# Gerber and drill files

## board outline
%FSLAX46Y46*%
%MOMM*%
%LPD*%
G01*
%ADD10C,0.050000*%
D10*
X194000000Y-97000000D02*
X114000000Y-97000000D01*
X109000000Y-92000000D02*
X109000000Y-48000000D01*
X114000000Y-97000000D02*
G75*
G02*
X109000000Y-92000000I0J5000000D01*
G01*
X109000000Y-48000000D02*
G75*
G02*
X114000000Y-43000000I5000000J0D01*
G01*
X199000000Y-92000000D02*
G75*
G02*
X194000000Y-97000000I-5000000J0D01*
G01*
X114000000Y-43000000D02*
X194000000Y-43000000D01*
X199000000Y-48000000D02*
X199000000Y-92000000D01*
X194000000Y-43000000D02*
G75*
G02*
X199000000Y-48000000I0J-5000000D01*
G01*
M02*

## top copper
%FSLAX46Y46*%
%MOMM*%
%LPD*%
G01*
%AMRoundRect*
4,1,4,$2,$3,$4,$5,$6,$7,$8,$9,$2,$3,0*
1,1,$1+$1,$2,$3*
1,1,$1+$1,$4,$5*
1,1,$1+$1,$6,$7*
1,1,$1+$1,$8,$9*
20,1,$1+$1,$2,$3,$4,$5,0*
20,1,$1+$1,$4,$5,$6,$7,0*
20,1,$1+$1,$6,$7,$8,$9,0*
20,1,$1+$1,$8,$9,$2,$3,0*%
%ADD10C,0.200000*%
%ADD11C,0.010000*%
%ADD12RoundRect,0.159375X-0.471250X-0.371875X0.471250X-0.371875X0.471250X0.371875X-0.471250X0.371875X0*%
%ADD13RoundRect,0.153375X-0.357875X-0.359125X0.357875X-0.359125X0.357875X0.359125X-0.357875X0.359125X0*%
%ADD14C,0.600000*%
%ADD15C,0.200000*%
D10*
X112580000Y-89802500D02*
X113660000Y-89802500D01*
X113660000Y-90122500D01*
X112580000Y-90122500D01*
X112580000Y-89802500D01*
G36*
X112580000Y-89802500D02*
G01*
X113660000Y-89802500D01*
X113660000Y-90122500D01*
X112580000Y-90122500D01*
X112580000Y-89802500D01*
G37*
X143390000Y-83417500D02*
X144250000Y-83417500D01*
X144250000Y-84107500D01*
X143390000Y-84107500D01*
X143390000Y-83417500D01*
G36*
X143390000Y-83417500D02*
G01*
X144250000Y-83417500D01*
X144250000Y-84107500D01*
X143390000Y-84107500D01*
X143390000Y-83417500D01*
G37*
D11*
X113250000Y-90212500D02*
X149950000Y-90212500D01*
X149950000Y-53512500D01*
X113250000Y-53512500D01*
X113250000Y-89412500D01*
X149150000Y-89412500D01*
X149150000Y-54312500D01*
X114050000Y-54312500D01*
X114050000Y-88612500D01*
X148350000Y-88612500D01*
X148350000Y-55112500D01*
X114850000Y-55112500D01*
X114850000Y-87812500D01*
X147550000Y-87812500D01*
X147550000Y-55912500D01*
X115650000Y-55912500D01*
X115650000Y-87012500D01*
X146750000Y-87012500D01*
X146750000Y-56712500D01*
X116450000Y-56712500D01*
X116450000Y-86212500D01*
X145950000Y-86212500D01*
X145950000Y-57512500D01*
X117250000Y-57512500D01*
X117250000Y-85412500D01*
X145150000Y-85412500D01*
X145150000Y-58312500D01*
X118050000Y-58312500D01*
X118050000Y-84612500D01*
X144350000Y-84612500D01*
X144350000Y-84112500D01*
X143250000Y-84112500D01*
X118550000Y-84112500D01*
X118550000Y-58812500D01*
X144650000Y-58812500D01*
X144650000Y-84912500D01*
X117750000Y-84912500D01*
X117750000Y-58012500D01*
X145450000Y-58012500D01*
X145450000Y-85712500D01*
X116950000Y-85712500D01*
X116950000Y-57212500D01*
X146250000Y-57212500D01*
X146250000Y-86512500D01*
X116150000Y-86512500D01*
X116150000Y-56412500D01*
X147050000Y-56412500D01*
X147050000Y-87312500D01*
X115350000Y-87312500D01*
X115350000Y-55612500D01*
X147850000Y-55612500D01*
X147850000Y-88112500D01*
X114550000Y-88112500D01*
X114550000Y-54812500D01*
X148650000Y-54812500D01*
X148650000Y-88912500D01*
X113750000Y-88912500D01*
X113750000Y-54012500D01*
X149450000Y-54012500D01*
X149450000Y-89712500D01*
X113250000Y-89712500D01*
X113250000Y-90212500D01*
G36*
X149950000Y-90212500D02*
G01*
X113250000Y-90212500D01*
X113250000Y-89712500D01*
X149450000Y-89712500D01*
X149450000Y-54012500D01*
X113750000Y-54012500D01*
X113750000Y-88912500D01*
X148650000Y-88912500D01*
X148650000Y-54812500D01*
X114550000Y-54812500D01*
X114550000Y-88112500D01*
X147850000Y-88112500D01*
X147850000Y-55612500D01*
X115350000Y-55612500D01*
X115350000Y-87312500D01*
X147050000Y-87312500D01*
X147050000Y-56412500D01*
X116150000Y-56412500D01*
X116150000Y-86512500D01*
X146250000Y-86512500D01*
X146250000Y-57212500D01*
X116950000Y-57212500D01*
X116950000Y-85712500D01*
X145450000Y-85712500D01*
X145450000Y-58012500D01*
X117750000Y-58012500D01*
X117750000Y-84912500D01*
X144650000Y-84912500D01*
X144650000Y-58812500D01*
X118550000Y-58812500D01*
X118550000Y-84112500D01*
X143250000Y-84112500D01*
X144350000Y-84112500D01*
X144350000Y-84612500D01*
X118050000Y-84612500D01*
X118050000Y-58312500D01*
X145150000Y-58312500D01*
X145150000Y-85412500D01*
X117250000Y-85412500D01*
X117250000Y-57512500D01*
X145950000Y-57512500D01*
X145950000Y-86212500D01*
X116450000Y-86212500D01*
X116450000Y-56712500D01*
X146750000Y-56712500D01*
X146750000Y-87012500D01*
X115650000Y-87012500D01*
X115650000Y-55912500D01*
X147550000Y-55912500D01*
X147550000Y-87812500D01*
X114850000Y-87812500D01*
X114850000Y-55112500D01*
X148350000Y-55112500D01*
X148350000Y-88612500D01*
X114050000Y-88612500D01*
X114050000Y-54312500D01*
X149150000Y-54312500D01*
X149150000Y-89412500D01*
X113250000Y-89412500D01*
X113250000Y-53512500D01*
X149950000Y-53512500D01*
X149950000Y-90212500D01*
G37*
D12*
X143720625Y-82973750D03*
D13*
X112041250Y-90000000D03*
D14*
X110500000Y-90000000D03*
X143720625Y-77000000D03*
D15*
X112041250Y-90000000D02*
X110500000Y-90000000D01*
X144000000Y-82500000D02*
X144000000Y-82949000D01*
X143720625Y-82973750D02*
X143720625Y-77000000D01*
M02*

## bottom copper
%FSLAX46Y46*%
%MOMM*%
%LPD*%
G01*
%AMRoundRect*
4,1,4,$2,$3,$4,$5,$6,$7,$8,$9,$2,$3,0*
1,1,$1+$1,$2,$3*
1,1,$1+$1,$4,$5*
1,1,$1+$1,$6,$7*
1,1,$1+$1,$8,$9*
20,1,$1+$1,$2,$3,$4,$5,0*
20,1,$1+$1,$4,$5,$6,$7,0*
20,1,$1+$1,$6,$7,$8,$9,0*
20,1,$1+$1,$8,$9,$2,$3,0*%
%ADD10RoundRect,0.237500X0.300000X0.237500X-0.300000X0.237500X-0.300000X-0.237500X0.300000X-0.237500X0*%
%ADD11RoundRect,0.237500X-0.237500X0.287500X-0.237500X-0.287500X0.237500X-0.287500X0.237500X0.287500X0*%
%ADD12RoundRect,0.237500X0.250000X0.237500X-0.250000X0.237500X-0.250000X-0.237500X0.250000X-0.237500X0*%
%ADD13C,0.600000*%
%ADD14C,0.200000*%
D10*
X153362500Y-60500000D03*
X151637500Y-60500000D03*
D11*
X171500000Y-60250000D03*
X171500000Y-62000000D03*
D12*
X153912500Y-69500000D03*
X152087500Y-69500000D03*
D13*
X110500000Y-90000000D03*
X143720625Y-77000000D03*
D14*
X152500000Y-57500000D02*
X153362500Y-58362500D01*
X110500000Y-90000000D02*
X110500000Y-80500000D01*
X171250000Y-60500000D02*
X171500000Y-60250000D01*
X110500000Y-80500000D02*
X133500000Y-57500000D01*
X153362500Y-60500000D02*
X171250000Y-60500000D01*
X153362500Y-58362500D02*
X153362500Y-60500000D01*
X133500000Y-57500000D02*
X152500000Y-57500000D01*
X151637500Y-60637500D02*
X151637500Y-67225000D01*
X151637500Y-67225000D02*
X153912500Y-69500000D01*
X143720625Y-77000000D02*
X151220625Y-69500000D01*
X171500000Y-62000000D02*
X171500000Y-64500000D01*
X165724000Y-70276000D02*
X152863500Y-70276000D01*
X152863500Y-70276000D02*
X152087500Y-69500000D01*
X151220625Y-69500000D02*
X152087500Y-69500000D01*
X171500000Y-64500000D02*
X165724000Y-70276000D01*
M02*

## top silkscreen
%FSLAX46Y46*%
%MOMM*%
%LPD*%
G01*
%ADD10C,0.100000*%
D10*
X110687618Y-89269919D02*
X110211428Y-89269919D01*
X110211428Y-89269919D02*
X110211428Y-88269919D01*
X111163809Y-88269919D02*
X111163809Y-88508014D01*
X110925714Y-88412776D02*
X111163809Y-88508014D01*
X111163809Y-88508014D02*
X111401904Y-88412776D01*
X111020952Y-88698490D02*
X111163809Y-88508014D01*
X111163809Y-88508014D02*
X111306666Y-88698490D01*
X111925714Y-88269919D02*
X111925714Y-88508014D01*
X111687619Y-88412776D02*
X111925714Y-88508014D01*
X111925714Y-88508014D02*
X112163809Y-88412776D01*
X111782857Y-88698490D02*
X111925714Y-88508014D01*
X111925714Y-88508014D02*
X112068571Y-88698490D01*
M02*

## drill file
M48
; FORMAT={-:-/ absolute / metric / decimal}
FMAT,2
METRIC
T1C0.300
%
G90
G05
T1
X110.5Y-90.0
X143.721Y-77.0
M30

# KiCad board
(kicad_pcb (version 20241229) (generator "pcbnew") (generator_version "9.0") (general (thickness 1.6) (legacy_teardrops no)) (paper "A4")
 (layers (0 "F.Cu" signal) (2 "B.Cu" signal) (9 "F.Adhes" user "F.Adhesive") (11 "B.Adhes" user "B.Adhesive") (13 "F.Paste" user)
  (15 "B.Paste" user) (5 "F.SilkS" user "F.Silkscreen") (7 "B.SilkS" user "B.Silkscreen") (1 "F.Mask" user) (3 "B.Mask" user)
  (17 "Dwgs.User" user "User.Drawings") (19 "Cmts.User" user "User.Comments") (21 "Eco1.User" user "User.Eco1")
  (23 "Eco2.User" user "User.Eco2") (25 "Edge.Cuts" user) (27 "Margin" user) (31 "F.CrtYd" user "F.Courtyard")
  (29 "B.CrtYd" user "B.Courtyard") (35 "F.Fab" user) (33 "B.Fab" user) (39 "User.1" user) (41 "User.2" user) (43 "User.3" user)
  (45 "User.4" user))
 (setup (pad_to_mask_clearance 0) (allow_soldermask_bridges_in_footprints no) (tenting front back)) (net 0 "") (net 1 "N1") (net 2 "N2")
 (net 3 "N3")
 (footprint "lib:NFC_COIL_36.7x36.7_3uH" (layer "F.Cu") (at 113.25 90.2125)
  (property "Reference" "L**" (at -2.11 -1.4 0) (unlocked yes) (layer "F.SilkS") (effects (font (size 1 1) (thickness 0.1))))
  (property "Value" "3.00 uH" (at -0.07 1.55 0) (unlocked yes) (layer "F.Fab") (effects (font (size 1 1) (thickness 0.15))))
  (fp_rect (start -0.67 -0.41) (end 0.41 -0.09) (stroke (width 0.2) (type solid)) (fill yes) (layer "F.Cu"))
  (fp_rect (start 30.14 -6.795) (end 31 -6.105) (stroke (width 0.2) (type solid)) (fill yes) (layer "F.Cu"))
  (fp_poly
   (pts (xy 0 0) (xy 36.7 0) (xy 36.7 -36.7) (xy 0 -36.7) (xy 0 -0.8) (xy 35.9 -0.8) (xy 35.9 -35.9) (xy 0.8 -35.9) (xy 0.8 -1.6)
    (xy 35.1 -1.6) (xy 35.1 -35.1) (xy 1.6 -35.1) (xy 1.6 -2.4) (xy 34.3 -2.4) (xy 34.3 -34.3) (xy 2.4 -34.3) (xy 2.4 -3.2) (xy 33.5 -3.2)
    (xy 33.5 -33.5) (xy 3.2 -33.5) (xy 3.2 -4) (xy 32.7 -4) (xy 32.7 -32.7) (xy 4 -32.7) (xy 4 -4.8) (xy 31.9 -4.8) (xy 31.9 -31.9)
    (xy 4.8 -31.9) (xy 4.8 -5.6) (xy 31.1 -5.6) (xy 31.1 -6.1) (xy 30 -6.1) (xy 5.3 -6.1) (xy 5.3 -31.4) (xy 31.4 -31.4) (xy 31.4 -5.3)
    (xy 4.5 -5.3) (xy 4.5 -32.2) (xy 32.2 -32.2) (xy 32.2 -4.5) (xy 3.7 -4.5) (xy 3.7 -33) (xy 33 -33) (xy 33 -3.7) (xy 2.9 -3.7)
    (xy 2.9 -33.8) (xy 33.8 -33.8) (xy 33.8 -2.9) (xy 2.1 -2.9) (xy 2.1 -34.6) (xy 34.6 -34.6) (xy 34.6 -2.1) (xy 1.3 -2.1) (xy 1.3 -35.4)
    (xy 35.4 -35.4) (xy 35.4 -1.3) (xy 0.5 -1.3) (xy 0.5 -36.2) (xy 36.2 -36.2) (xy 36.2 -0.5) (xy 0 -0.5))
   (stroke (width 0.01) (type solid)) (fill yes) (layer "F.Cu"))
  (pad "1" smd roundrect (at 30.470625 -7.23875) (size 1.26125 1.0625) (layers "F.Cu" "F.Mask" "F.Paste") (roundrect_rratio 0.15)
   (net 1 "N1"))
  (pad "2" smd roundrect (at -1.20875 -0.2125) (size 1.0225 1.025) (layers "F.Cu" "F.Mask" "F.Paste") (roundrect_rratio 0.15) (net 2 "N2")))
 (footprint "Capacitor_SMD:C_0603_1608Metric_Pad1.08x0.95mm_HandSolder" (layer "B.Cu") (at 152.5 60.5 180)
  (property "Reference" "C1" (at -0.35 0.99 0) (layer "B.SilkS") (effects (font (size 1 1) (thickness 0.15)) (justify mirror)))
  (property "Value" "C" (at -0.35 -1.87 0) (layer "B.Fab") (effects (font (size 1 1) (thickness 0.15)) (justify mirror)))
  (pad "1" smd roundrect (at -0.8625 0 180) (size 1.075 0.95) (layers "B.Cu" "B.Mask" "B.Paste") (roundrect_rratio 0.25) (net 2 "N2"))
  (pad "2" smd roundrect (at 0.8625 0 180) (size 1.075 0.95) (layers "B.Cu" "B.Mask" "B.Paste") (roundrect_rratio 0.25) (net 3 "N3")))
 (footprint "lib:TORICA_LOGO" (layer "B.Cu") (at 176 54.5 180)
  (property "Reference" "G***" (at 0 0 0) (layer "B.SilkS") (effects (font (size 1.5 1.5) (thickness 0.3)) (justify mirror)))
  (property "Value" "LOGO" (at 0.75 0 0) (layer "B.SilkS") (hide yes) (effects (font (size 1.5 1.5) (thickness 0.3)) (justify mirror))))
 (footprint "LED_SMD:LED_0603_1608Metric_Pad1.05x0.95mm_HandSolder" (layer "B.Cu") (at 171.5 61.125 -90)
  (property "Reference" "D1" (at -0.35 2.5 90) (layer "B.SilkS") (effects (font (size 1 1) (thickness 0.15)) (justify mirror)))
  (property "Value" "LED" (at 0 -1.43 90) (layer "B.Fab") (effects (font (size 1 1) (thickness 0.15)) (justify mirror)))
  (pad "1" smd roundrect (at -0.875 0 270) (size 1.05 0.95) (layers "B.Cu" "B.Mask" "B.Paste") (roundrect_rratio 0.25) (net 2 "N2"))
  (pad "2" smd roundrect (at 0.875 0 270) (size 1.05 0.95) (layers "B.Cu" "B.Mask" "B.Paste") (roundrect_rratio 0.25) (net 1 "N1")))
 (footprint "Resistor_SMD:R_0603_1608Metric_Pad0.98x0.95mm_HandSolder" (layer "B.Cu") (at 153 69.5 180)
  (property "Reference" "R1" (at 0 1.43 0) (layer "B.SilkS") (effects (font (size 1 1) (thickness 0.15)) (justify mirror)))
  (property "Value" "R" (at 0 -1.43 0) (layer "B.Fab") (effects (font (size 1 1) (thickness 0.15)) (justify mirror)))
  (pad "1" smd roundrect (at -0.9125 0 180) (size 0.975 0.95) (layers "B.Cu" "B.Mask" "B.Paste") (roundrect_rratio 0.25) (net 3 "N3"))
  (pad "2" smd roundrect (at 0.9125 0 180) (size 0.975 0.95) (layers "B.Cu" "B.Mask" "B.Paste") (roundrect_rratio 0.25) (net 1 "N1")))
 (gr_line (start 194 97) (end 114 97) (stroke (width 0.05) (type default)) (layer "Edge.Cuts"))
 (gr_line (start 109 92) (end 109 48) (stroke (width 0.05) (type default)) (layer "Edge.Cuts"))
 (gr_arc (start 114 97) (mid 110.464466 95.535534) (end 109 92) (stroke (width 0.05) (type default)) (layer "Edge.Cuts"))
 (gr_arc (start 109 48) (mid 110.464466 44.464466) (end 114 43) (stroke (width 0.05) (type default)) (layer "Edge.Cuts"))
 (gr_arc (start 199 92) (mid 197.535534 95.535534) (end 194 97) (stroke (width 0.05) (type default)) (layer "Edge.Cuts"))
 (gr_line (start 114 43) (end 194 43) (stroke (width 0.05) (type default)) (layer "Edge.Cuts"))
 (gr_line (start 199 48) (end 199 92) (stroke (width 0.05) (type default)) (layer "Edge.Cuts"))
 (gr_arc (start 194 43) (mid 197.535534 44.464466) (end 199 48) (stroke (width 0.05) (type default)) (layer "Edge.Cuts"))
 (segment (start 112.04125 90) (end 110.5 90) (width 0.2) (layer "F.Cu") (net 2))
 (via (at 110.5 90) (size 0.6) (drill 0.3) (layers "F.Cu" "B.Cu") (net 2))
 (segment (start 152.5 57.5) (end 153.3625 58.3625) (width 0.2) (layer "B.Cu") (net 2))
 (segment (start 110.5 90) (end 110.5 80.5) (width 0.2) (layer "B.Cu") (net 2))
 (segment (start 171.25 60.5) (end 171.5 60.25) (width 0.2) (layer "B.Cu") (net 2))
 (segment (start 110.5 80.5) (end 133.5 57.5) (width 0.2) (layer "B.Cu") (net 2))
 (segment (start 153.3625 60.5) (end 171.25 60.5) (width 0.2) (layer "B.Cu") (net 2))
 (segment (start 153.3625 58.3625) (end 153.3625 60.5) (width 0.2) (layer "B.Cu") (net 2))
 (segment (start 133.5 57.5) (end 152.5 57.5) (width 0.2) (layer "B.Cu") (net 2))
 (segment (start 151.6375 60.6375) (end 151.6375 67.225) (width 0.2) (layer "B.Cu") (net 3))
 (segment (start 151.6375 67.225) (end 153.9125 69.5) (width 0.2) (layer "B.Cu") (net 3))
 (segment (start 144 82.5) (end 144 82.949) (width 0.2) (layer "F.Cu") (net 1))
 (segment (start 143.720625 82.97375) (end 143.720625 77) (width 0.2) (layer "F.Cu") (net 1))
 (via (at 143.720625 77) (size 0.6) (drill 0.3) (layers "F.Cu" "B.Cu") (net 1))
 (segment (start 143.720625 77) (end 151.220625 69.5) (width 0.2) (layer "B.Cu") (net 1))
 (segment (start 171.5 62) (end 171.5 64.5) (width 0.2) (layer "B.Cu") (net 1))
 (segment (start 165.724 70.276) (end 152.8635 70.276) (width 0.2) (layer "B.Cu") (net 1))
 (segment (start 152.8635 70.276) (end 152.0875 69.5) (width 0.2) (layer "B.Cu") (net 1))
 (segment (start 151.220625 69.5) (end 152.0875 69.5) (width 0.2) (layer "B.Cu") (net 1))
 (segment (start 171.5 64.5) (end 165.724 70.276) (width 0.2) (layer "B.Cu") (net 1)))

